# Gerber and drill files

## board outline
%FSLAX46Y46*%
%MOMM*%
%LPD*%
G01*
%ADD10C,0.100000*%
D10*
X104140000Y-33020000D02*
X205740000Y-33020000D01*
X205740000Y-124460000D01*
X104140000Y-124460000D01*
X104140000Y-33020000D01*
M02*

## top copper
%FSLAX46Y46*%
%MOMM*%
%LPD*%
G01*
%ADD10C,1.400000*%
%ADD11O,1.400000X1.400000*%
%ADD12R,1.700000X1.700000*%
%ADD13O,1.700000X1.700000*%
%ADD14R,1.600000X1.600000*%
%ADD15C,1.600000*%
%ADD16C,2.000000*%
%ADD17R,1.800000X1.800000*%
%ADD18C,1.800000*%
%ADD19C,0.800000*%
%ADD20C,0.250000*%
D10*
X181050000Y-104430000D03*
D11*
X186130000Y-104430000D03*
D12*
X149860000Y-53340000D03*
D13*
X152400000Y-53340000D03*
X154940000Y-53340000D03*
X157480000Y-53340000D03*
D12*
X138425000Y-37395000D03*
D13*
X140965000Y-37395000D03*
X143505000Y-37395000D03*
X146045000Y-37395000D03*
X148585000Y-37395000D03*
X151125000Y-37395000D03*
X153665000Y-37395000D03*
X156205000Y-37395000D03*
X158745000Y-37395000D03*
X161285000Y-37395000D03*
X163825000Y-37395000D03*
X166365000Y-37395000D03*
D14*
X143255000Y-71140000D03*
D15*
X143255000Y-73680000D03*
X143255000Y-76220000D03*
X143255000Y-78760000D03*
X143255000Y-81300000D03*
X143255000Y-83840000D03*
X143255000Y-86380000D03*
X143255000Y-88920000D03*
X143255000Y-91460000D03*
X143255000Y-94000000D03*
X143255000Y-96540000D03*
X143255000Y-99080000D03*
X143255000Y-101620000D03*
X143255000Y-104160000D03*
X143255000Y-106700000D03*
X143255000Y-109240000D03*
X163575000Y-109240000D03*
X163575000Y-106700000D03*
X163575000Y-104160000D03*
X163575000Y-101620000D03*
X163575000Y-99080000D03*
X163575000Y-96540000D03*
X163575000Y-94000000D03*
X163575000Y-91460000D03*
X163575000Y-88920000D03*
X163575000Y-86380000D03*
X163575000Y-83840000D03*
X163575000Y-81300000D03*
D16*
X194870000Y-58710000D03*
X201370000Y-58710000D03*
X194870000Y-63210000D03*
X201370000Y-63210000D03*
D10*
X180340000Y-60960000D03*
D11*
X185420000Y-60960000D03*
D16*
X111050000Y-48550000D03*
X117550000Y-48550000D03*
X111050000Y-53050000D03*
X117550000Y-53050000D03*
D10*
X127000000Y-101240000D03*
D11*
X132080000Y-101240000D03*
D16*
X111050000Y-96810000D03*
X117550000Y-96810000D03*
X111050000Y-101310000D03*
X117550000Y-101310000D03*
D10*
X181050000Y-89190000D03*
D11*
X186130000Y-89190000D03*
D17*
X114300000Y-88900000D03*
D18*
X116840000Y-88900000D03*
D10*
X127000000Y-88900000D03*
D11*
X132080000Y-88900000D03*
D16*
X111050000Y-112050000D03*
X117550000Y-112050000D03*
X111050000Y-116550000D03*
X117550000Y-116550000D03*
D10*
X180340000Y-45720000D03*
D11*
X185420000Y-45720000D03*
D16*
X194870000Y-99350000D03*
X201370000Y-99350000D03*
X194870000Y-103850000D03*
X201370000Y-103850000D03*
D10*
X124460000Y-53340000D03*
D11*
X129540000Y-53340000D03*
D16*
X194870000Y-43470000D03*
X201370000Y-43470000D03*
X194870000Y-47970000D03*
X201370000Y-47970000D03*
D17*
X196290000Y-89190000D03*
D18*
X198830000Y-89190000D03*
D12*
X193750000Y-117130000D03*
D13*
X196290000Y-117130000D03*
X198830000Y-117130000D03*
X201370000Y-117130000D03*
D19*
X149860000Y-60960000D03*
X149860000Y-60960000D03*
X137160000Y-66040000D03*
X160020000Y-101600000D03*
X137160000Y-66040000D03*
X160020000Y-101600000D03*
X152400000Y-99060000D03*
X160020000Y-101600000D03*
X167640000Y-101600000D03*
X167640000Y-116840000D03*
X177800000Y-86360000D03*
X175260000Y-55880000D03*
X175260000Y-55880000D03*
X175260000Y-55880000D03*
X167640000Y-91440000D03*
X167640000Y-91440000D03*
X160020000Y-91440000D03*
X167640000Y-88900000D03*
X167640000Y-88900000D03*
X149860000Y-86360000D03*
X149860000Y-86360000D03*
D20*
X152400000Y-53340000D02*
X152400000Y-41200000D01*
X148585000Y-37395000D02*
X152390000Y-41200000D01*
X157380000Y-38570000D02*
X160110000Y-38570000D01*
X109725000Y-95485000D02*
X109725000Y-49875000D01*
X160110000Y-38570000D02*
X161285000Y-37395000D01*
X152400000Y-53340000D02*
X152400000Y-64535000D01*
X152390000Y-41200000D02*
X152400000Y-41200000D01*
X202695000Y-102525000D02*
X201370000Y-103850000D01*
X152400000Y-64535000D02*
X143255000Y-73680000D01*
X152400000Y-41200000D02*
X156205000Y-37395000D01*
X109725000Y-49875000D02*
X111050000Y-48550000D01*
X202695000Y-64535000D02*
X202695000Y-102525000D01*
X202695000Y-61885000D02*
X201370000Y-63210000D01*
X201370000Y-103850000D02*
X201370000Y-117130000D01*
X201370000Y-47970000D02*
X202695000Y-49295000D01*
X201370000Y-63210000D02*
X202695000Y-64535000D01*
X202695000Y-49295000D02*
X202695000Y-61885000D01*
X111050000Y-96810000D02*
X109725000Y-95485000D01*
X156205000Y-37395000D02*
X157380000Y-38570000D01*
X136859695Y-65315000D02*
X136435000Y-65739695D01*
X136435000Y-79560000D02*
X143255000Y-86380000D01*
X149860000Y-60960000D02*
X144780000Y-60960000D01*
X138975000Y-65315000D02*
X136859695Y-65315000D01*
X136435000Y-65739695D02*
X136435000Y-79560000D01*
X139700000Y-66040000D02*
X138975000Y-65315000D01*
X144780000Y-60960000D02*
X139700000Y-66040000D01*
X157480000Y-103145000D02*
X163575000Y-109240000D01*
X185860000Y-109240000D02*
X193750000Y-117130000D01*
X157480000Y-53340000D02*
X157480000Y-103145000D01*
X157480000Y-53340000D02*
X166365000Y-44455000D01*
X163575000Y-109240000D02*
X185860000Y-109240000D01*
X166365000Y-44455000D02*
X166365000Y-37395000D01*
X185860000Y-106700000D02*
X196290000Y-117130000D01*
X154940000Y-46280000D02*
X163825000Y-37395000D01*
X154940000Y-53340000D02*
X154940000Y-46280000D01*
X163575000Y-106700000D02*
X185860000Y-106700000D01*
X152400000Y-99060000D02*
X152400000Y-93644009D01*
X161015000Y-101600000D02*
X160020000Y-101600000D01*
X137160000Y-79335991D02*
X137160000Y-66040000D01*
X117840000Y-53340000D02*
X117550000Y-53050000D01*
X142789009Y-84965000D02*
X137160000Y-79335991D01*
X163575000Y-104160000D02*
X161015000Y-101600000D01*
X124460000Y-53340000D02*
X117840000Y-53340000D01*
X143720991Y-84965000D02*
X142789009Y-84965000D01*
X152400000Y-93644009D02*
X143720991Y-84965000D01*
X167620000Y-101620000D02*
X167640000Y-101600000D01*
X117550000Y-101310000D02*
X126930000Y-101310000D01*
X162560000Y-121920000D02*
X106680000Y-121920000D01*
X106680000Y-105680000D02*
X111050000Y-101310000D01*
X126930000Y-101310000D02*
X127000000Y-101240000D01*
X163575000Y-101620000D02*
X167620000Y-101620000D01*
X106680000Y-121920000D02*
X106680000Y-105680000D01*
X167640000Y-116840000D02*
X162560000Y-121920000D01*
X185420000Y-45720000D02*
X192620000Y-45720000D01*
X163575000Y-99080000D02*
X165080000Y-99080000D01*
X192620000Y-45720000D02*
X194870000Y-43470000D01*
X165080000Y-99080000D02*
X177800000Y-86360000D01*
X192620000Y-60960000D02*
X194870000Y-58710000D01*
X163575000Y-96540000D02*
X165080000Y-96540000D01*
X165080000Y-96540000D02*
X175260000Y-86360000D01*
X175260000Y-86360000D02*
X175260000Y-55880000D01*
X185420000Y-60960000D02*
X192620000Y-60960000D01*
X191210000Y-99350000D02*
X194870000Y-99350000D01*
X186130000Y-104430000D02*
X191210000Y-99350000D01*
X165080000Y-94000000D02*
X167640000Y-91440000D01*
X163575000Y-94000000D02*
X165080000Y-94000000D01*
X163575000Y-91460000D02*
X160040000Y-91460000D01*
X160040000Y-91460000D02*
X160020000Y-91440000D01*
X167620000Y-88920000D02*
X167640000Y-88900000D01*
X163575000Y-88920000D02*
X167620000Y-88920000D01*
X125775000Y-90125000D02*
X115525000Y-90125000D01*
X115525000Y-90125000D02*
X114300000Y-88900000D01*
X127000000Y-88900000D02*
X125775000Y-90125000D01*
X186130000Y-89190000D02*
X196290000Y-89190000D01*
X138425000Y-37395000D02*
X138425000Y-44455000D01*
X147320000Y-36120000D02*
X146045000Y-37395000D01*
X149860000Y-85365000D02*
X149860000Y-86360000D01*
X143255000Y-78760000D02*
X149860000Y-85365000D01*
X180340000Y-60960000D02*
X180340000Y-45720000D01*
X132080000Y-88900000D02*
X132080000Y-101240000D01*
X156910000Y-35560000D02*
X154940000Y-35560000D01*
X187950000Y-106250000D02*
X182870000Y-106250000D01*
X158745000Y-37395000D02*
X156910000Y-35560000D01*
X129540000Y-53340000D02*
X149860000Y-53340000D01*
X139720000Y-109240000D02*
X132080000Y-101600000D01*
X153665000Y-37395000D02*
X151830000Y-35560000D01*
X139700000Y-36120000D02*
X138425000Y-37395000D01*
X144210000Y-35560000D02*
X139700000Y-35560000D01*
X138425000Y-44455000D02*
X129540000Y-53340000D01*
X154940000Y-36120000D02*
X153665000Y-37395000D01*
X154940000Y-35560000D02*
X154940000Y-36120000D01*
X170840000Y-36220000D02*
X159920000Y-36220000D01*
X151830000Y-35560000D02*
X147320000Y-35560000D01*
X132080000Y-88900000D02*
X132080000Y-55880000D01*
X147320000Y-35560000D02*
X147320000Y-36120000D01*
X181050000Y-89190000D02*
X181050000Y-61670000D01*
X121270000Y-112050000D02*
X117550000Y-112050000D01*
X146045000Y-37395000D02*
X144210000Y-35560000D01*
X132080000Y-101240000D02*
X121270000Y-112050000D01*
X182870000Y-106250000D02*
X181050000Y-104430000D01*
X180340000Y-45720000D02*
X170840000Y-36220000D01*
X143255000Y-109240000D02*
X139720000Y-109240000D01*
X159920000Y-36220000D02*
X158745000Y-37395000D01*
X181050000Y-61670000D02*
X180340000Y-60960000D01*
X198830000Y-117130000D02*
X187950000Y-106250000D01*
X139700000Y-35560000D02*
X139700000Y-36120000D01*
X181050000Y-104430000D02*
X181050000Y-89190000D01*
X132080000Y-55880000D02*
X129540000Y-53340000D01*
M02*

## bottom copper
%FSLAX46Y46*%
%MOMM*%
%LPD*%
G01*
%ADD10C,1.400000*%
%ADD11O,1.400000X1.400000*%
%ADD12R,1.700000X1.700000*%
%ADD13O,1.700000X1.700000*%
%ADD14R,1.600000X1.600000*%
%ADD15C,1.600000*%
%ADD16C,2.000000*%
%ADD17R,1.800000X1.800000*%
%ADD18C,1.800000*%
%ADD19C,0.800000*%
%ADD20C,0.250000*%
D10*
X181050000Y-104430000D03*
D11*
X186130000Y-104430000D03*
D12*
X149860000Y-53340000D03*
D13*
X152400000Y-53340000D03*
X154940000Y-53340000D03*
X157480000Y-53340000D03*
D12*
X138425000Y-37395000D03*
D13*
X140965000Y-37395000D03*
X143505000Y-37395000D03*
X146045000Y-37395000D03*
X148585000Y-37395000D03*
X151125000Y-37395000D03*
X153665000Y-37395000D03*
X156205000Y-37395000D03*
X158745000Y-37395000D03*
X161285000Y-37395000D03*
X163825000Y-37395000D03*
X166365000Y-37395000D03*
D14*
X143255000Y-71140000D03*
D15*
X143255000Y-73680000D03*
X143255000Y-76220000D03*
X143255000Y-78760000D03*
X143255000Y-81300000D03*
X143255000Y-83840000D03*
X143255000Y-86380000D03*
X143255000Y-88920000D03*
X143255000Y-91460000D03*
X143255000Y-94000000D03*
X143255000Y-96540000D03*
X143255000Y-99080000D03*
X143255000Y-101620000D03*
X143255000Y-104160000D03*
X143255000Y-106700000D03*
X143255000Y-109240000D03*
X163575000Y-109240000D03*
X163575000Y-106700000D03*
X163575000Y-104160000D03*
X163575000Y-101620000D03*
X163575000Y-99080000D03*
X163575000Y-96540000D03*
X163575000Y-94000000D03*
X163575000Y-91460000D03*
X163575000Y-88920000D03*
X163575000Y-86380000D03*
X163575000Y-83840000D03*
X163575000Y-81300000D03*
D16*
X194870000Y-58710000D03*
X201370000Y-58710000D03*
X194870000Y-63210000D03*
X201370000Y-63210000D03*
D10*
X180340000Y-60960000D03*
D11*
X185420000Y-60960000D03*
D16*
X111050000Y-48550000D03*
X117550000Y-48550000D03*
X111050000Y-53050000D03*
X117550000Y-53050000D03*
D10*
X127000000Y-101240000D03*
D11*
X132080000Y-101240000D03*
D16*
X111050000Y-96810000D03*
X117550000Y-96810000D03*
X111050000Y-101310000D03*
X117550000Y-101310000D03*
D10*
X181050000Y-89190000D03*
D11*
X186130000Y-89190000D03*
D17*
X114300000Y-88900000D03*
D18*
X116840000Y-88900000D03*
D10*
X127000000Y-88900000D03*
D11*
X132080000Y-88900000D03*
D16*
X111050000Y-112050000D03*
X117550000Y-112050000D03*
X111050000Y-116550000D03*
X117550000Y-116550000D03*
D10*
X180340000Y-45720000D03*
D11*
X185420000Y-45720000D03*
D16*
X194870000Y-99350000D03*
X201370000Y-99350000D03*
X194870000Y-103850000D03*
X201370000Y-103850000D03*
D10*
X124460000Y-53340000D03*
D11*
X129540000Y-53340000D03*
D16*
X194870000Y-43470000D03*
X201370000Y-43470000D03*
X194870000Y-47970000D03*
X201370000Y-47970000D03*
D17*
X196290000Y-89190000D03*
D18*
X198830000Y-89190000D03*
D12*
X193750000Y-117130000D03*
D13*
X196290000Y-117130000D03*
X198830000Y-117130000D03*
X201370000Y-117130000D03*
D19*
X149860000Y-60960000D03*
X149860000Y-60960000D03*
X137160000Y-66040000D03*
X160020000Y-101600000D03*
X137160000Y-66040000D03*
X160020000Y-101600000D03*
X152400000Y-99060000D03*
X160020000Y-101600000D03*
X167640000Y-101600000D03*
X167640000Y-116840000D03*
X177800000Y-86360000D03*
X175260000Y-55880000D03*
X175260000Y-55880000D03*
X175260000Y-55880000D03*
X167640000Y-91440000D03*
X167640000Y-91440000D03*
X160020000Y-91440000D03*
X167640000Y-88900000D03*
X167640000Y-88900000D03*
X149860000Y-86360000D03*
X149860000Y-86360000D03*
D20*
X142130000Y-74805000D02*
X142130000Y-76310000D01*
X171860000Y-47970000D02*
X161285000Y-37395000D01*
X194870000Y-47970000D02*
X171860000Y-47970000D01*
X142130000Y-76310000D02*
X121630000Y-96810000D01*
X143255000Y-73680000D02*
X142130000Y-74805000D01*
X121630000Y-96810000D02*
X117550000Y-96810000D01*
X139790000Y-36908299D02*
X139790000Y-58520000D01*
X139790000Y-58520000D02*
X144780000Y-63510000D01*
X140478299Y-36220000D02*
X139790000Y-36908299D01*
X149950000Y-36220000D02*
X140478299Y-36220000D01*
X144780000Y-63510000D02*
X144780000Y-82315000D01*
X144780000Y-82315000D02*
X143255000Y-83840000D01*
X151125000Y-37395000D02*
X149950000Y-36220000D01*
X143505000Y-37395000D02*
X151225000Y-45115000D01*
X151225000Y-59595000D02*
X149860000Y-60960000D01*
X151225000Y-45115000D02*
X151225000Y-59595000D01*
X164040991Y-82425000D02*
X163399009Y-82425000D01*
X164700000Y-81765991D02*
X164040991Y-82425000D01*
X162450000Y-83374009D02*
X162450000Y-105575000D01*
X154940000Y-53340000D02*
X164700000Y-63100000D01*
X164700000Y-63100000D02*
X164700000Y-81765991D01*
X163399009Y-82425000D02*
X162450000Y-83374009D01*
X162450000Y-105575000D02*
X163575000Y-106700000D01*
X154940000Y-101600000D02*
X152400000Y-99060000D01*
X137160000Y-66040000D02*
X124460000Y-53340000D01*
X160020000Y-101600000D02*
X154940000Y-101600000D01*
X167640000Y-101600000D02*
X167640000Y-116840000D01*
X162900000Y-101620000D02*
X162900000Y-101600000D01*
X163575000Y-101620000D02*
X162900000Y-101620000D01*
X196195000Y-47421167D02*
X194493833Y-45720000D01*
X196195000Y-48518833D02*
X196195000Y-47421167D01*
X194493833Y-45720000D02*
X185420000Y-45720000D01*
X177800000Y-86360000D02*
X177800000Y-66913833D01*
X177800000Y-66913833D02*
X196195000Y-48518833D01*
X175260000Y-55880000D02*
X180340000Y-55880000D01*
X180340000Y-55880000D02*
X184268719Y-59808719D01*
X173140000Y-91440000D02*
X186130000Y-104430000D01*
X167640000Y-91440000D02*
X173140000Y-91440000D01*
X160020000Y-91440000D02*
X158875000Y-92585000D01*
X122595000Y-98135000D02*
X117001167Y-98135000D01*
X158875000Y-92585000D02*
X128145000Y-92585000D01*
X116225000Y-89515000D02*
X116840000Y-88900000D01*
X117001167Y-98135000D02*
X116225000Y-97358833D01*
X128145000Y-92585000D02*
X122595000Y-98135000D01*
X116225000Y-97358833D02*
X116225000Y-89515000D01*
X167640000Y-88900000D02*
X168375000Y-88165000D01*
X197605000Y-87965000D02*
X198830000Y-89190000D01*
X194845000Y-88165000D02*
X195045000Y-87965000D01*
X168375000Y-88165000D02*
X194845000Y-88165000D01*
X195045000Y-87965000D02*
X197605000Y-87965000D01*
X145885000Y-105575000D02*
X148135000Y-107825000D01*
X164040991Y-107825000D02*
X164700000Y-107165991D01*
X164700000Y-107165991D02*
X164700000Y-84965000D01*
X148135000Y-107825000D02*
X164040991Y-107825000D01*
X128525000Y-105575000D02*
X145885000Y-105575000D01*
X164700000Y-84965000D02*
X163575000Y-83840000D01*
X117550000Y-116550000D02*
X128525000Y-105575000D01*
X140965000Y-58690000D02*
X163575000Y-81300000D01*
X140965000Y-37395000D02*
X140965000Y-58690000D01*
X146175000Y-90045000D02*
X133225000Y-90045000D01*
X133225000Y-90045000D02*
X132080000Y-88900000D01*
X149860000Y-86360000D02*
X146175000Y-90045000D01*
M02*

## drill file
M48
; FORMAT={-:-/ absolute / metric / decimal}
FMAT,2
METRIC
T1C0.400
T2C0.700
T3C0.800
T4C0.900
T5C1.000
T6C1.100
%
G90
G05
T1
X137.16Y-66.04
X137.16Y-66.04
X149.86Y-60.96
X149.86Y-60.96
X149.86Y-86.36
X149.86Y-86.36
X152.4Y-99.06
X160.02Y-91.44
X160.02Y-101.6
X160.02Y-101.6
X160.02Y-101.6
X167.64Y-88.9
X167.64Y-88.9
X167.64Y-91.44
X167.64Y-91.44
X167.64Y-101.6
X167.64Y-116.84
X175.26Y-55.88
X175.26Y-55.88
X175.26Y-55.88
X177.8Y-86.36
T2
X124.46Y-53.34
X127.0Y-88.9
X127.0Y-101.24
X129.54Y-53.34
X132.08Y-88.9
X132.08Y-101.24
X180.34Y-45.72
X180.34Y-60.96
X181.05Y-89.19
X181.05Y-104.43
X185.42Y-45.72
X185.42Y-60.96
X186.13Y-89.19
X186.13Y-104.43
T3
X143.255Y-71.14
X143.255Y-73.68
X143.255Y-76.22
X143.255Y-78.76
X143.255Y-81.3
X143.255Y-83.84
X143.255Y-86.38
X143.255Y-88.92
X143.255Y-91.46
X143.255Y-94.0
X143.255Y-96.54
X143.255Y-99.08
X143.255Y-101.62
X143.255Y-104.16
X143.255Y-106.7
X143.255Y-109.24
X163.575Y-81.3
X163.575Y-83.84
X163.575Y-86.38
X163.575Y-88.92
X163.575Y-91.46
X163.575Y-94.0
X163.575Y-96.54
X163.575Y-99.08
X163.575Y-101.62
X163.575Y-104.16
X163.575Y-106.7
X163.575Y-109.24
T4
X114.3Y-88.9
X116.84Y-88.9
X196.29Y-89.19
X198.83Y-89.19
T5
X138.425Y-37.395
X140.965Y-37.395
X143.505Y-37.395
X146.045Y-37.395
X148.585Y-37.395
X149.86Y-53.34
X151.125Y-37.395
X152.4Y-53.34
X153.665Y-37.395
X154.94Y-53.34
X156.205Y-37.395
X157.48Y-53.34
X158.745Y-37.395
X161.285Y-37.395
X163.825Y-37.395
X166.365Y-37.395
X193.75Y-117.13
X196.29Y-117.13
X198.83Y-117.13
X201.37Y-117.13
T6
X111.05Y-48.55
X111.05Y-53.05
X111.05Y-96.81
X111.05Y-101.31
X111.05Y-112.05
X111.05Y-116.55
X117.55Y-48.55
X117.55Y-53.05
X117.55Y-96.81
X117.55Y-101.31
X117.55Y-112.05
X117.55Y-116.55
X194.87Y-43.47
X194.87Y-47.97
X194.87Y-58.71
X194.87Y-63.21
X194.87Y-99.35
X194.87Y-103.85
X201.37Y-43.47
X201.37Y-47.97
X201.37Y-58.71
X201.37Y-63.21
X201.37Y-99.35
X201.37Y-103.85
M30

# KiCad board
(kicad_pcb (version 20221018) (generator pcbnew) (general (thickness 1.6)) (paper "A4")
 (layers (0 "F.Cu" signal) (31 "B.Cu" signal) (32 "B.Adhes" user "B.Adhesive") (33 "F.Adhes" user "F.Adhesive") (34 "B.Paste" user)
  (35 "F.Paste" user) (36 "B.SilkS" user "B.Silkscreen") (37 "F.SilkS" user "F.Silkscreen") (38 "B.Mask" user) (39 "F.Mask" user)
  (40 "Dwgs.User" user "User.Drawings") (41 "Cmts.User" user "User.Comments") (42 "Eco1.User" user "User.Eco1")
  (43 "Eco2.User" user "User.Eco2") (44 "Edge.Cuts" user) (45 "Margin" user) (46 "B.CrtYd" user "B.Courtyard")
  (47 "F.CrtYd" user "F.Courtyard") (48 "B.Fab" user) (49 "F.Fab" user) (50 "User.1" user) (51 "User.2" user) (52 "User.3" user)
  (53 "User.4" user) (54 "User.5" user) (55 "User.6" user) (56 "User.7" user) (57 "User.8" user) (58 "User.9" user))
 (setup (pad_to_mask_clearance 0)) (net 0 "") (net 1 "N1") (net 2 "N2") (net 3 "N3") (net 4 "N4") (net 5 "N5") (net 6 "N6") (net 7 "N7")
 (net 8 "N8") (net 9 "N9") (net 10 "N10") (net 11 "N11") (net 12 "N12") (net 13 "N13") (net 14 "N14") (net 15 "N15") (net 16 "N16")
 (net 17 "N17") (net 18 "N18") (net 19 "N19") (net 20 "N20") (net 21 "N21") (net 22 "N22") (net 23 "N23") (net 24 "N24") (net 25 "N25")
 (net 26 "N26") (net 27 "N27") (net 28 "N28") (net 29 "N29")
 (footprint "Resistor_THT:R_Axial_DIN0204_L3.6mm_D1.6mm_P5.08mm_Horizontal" (layer "F.Cu") (at 181.05 104.43)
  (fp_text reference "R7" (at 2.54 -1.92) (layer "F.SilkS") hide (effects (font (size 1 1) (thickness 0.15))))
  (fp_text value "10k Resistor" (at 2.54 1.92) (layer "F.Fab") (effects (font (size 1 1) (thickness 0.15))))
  (pad "1" thru_hole circle (at 0 0) (size 1.4 1.4) (drill 0.7) (layers "*.Cu" "*.Mask") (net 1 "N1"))
  (pad "2" thru_hole oval (at 5.08 0) (size 1.4 1.4) (drill 0.7) (layers "*.Cu" "*.Mask") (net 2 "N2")))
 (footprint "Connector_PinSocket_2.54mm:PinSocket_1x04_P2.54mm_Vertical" (layer "F.Cu") (at 149.86 53.34 90)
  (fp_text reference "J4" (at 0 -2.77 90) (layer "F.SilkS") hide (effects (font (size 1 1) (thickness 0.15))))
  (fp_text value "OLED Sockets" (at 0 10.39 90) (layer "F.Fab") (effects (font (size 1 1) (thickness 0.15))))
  (pad "1" thru_hole rect (at 0 0 90) (size 1.7 1.7) (drill 1) (layers "*.Cu" "*.Mask") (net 1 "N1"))
  (pad "2" thru_hole oval (at 0 2.54 90) (size 1.7 1.7) (drill 1) (layers "*.Cu" "*.Mask") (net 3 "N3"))
  (pad "3" thru_hole oval (at 0 5.08 90) (size 1.7 1.7) (drill 1) (layers "*.Cu" "*.Mask") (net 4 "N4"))
  (pad "4" thru_hole oval (at 0 7.62 90) (size 1.7 1.7) (drill 1) (layers "*.Cu" "*.Mask") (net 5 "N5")))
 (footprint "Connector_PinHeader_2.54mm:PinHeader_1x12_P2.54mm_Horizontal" (layer "F.Cu") (at 138.425 37.395 90)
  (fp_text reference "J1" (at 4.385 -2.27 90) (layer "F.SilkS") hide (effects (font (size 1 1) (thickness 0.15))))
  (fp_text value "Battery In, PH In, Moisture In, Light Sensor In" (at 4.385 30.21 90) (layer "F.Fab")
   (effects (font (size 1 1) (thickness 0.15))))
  (pad "1" thru_hole rect (at 0 0 90) (size 1.7 1.7) (drill 1) (layers "*.Cu" "*.Mask") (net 1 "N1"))
  (pad "2" thru_hole oval (at 0 2.54 90) (size 1.7 1.7) (drill 1) (layers "*.Cu" "*.Mask") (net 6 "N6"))
  (pad "3" thru_hole oval (at 0 5.08 90) (size 1.7 1.7) (drill 1) (layers "*.Cu" "*.Mask") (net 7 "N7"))
  (pad "4" thru_hole oval (at 0 7.62 90) (size 1.7 1.7) (drill 1) (layers "*.Cu" "*.Mask") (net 1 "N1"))
  (pad "5" thru_hole oval (at 0 10.16 90) (size 1.7 1.7) (drill 1) (layers "*.Cu" "*.Mask") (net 3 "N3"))
  (pad "6" thru_hole oval (at 0 12.7 90) (size 1.7 1.7) (drill 1) (layers "*.Cu" "*.Mask") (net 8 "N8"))
  (pad "7" thru_hole oval (at 0 15.24 90) (size 1.7 1.7) (drill 1) (layers "*.Cu" "*.Mask") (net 1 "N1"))
  (pad "8" thru_hole oval (at 0 17.78 90) (size 1.7 1.7) (drill 1) (layers "*.Cu" "*.Mask") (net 3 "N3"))
  (pad "9" thru_hole oval (at 0 20.32 90) (size 1.7 1.7) (drill 1) (layers "*.Cu" "*.Mask") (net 1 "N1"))
  (pad "10" thru_hole oval (at 0 22.86 90) (size 1.7 1.7) (drill 1) (layers "*.Cu" "*.Mask") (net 3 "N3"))
  (pad "11" thru_hole oval (at 0 25.4 90) (size 1.7 1.7) (drill 1) (layers "*.Cu" "*.Mask") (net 4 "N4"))
  (pad "12" thru_hole oval (at 0 27.94 90) (size 1.7 1.7) (drill 1) (layers "*.Cu" "*.Mask") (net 5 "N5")))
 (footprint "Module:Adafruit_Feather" (layer "F.Cu") (at 143.255 71.14)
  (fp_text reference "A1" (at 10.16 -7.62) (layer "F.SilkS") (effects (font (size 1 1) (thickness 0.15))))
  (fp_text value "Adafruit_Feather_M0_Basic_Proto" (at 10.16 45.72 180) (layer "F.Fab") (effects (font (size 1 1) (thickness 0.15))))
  (pad "1" thru_hole rect (at 0 0 180) (size 1.6 1.6) (drill 0.8) (layers "*.Cu" "*.Mask") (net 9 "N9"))
  (pad "2" thru_hole circle (at 0 2.54 180) (size 1.6 1.6) (drill 0.8) (layers "*.Cu" "*.Mask") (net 3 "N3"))
  (pad "3" thru_hole circle (at 0 5.08 180) (size 1.6 1.6) (drill 0.8) (layers "*.Cu" "*.Mask") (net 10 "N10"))
  (pad "4" thru_hole circle (at 0 7.62 180) (size 1.6 1.6) (drill 0.8) (layers "*.Cu" "*.Mask") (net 1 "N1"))
  (pad "5" thru_hole circle (at 0 10.16 180) (size 1.6 1.6) (drill 0.8) (layers "*.Cu" "*.Mask") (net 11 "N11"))
  (pad "6" thru_hole circle (at 0 12.7 180) (size 1.6 1.6) (drill 0.8) (layers "*.Cu" "*.Mask") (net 8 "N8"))
  (pad "7" thru_hole circle (at 0 15.24 180) (size 1.6 1.6) (drill 0.8) (layers "*.Cu" "*.Mask") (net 7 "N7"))
  (pad "8" thru_hole circle (at 0 17.78 180) (size 1.6 1.6) (drill 0.8) (layers "*.Cu" "*.Mask") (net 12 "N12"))
  (pad "9" thru_hole circle (at 0 20.32 180) (size 1.6 1.6) (drill 0.8) (layers "*.Cu" "*.Mask") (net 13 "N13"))
  (pad "10" thru_hole circle (at 0 22.86 180) (size 1.6 1.6) (drill 0.8) (layers "*.Cu" "*.Mask") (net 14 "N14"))
  (pad "11" thru_hole circle (at 0 25.4 180) (size 1.6 1.6) (drill 0.8) (layers "*.Cu" "*.Mask") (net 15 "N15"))
  (pad "12" thru_hole circle (at 0 27.94 180) (size 1.6 1.6) (drill 0.8) (layers "*.Cu" "*.Mask") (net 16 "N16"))
  (pad "13" thru_hole circle (at 0 30.48 180) (size 1.6 1.6) (drill 0.8) (layers "*.Cu" "*.Mask") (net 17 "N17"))
  (pad "14" thru_hole circle (at 0 33.02 180) (size 1.6 1.6) (drill 0.8) (layers "*.Cu" "*.Mask") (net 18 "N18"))
  (pad "15" thru_hole circle (at 0 35.56 180) (size 1.6 1.6) (drill 0.8) (layers "*.Cu" "*.Mask") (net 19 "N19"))
  (pad "16" thru_hole circle (at 0 38.1 180) (size 1.6 1.6) (drill 0.8) (layers "*.Cu" "*.Mask") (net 1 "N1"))
  (pad "17" thru_hole circle (at 20.32 38.1 180) (size 1.6 1.6) (drill 0.8) (layers "*.Cu" "*.Mask") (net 5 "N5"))
  (pad "18" thru_hole circle (at 20.32 35.56 180) (size 1.6 1.6) (drill 0.8) (layers "*.Cu" "*.Mask") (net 4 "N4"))
  (pad "19" thru_hole circle (at 20.32 33.02 180) (size 1.6 1.6) (drill 0.8) (layers "*.Cu" "*.Mask") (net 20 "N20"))
  (pad "20" thru_hole circle (at 20.32 30.48 180) (size 1.6 1.6) (drill 0.8) (layers "*.Cu" "*.Mask") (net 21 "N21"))
  (pad "21" thru_hole circle (at 20.32 27.94 180) (size 1.6 1.6) (drill 0.8) (layers "*.Cu" "*.Mask") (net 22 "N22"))
  (pad "22" thru_hole circle (at 20.32 25.4 180) (size 1.6 1.6) (drill 0.8) (layers "*.Cu" "*.Mask") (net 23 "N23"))
  (pad "23" thru_hole circle (at 20.32 22.86 180) (size 1.6 1.6) (drill 0.8) (layers "*.Cu" "*.Mask") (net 2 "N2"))
  (pad "24" thru_hole circle (at 20.32 20.32 180) (size 1.6 1.6) (drill 0.8) (layers "*.Cu" "*.Mask") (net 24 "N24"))
  (pad "25" thru_hole circle (at 20.32 17.78 180) (size 1.6 1.6) (drill 0.8) (layers "*.Cu" "*.Mask") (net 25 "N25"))
  (pad "26" thru_hole circle (at 20.32 15.24 180) (size 1.6 1.6) (drill 0.8) (layers "*.Cu" "*.Mask") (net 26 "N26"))
  (pad "27" thru_hole circle (at 20.32 12.7 180) (size 1.6 1.6) (drill 0.8) (layers "*.Cu" "*.Mask") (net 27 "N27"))
  (pad "28" thru_hole circle (at 20.32 10.16 180) (size 1.6 1.6) (drill 0.8) (layers "*.Cu" "*.Mask") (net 6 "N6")))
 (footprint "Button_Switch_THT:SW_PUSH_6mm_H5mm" (layer "F.Cu") (at 194.87 58.71)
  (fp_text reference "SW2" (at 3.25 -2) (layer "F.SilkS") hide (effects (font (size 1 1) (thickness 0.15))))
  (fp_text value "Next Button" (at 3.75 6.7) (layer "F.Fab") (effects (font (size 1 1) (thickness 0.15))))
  (pad "1" thru_hole circle (at 0 0 90) (size 2 2) (drill 1.1) (layers "*.Cu" "*.Mask") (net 23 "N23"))
  (pad "1" thru_hole circle (at 6.5 0 90) (size 2 2) (drill 1.1) (layers "*.Cu" "*.Mask") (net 23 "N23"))
  (pad "2" thru_hole circle (at 0 4.5 90) (size 2 2) (drill 1.1) (layers "*.Cu" "*.Mask") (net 3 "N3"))
  (pad "2" thru_hole circle (at 6.5 4.5 90) (size 2 2) (drill 1.1) (layers "*.Cu" "*.Mask") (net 3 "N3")))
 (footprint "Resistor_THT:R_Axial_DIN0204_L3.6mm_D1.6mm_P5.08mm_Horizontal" (layer "F.Cu") (at 180.34 60.96)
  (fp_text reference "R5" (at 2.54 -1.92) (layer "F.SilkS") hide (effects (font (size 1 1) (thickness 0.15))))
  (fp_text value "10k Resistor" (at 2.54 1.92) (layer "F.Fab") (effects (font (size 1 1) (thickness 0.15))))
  (pad "1" thru_hole circle (at 0 0) (size 1.4 1.4) (drill 0.7) (layers "*.Cu" "*.Mask") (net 1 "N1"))
  (pad "2" thru_hole oval (at 5.08 0) (size 1.4 1.4) (drill 0.7) (layers "*.Cu" "*.Mask") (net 23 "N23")))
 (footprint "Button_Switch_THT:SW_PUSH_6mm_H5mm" (layer "F.Cu") (at 111.05 48.55)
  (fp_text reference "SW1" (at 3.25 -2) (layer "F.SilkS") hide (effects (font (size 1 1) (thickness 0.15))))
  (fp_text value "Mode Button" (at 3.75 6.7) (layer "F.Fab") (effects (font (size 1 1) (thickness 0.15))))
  (pad "1" thru_hole circle (at 0 0 90) (size 2 2) (drill 1.1) (layers "*.Cu" "*.Mask") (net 3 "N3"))
  (pad "1" thru_hole circle (at 6.5 0 90) (size 2 2) (drill 1.1) (layers "*.Cu" "*.Mask") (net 3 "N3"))
  (pad "2" thru_hole circle (at 0 4.5 90) (size 2 2) (drill 1.1) (layers "*.Cu" "*.Mask") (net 20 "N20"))
  (pad "2" thru_hole circle (at 6.5 4.5 90) (size 2 2) (drill 1.1) (layers "*.Cu" "*.Mask") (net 20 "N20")))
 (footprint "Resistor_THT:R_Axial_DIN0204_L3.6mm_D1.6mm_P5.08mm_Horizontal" (layer "F.Cu") (at 127 101.24)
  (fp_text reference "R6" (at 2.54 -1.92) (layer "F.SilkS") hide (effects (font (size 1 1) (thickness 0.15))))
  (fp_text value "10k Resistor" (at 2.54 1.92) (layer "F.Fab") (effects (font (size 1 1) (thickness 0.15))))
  (pad "1" thru_hole circle (at 0 0) (size 1.4 1.4) (drill 0.7) (layers "*.Cu" "*.Mask") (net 21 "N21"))
  (pad "2" thru_hole oval (at 5.08 0) (size 1.4 1.4) (drill 0.7) (layers "*.Cu" "*.Mask") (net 1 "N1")))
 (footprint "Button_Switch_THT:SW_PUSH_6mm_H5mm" (layer "F.Cu") (at 111.05 96.81)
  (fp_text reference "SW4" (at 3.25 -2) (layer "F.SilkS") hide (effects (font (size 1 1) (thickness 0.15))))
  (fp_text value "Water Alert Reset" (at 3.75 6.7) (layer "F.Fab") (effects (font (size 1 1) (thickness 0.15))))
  (pad "1" thru_hole circle (at 0 0 90) (size 2 2) (drill 1.1) (layers "*.Cu" "*.Mask") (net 3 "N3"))
  (pad "1" thru_hole circle (at 6.5 0 90) (size 2 2) (drill 1.1) (layers "*.Cu" "*.Mask") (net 3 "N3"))
  (pad "2" thru_hole circle (at 0 4.5 90) (size 2 2) (drill 1.1) (layers "*.Cu" "*.Mask") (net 21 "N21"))
  (pad "2" thru_hole circle (at 6.5 4.5 90) (size 2 2) (drill 1.1) (layers "*.Cu" "*.Mask") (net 21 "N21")))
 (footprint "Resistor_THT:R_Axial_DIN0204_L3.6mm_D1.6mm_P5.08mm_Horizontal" (layer "F.Cu") (at 181.05 89.19)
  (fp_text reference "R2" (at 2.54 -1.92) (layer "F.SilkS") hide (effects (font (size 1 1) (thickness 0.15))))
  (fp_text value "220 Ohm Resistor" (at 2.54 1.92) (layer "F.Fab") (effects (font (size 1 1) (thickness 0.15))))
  (pad "1" thru_hole circle (at 0 0) (size 1.4 1.4) (drill 0.7) (layers "*.Cu" "*.Mask") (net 1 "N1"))
  (pad "2" thru_hole oval (at 5.08 0) (size 1.4 1.4) (drill 0.7) (layers "*.Cu" "*.Mask") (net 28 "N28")))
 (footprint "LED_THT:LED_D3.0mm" (layer "F.Cu") (at 114.3 88.9)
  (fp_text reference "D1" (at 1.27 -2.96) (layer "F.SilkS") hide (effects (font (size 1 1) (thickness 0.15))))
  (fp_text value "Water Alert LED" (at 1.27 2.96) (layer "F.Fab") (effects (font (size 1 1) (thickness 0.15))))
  (pad "1" thru_hole rect (at 0 0) (size 1.8 1.8) (drill 0.9) (layers "*.Cu" "*.Mask") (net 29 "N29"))
  (pad "2" thru_hole circle (at 2.54 0) (size 1.8 1.8) (drill 0.9) (layers "*.Cu" "*.Mask") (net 24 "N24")))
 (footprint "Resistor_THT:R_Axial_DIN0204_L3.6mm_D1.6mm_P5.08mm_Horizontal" (layer "F.Cu") (at 127 88.9)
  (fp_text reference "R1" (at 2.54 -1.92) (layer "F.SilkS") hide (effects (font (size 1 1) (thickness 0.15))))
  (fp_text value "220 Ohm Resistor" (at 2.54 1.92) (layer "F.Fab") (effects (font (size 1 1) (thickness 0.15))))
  (pad "1" thru_hole circle (at 0 0) (size 1.4 1.4) (drill 0.7) (layers "*.Cu" "*.Mask") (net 29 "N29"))
  (pad "2" thru_hole oval (at 5.08 0) (size 1.4 1.4) (drill 0.7) (layers "*.Cu" "*.Mask") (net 1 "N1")))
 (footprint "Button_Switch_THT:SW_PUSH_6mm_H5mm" (layer "F.Cu") (at 111.05 112.05)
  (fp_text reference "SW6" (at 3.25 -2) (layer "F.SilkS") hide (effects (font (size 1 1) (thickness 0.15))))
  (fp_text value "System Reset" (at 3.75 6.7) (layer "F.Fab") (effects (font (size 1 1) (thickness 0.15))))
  (pad "1" thru_hole circle (at 0 0 90) (size 2 2) (drill 1.1) (layers "*.Cu" "*.Mask") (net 1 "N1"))
  (pad "1" thru_hole circle (at 6.5 0 90) (size 2 2) (drill 1.1) (layers "*.Cu" "*.Mask") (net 1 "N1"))
  (pad "2" thru_hole circle (at 0 4.5 90) (size 2 2) (drill 1.1) (layers "*.Cu" "*.Mask") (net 27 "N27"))
  (pad "2" thru_hole circle (at 6.5 4.5 90) (size 2 2) (drill 1.1) (layers "*.Cu" "*.Mask") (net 27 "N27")))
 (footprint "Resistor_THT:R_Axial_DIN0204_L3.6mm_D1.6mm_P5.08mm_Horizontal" (layer "F.Cu") (at 180.34 45.72)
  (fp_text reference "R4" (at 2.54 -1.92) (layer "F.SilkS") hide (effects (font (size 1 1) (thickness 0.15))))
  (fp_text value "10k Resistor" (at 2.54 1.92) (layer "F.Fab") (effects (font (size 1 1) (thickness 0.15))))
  (pad "1" thru_hole circle (at 0 0) (size 1.4 1.4) (drill 0.7) (layers "*.Cu" "*.Mask") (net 1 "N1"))
  (pad "2" thru_hole oval (at 5.08 0) (size 1.4 1.4) (drill 0.7) (layers "*.Cu" "*.Mask") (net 22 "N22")))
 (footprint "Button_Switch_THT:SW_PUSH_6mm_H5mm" (layer "F.Cu") (at 194.87 99.35)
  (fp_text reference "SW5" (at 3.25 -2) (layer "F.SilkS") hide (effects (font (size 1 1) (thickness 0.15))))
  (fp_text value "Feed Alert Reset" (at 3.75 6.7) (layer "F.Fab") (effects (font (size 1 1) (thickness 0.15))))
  (pad "1" thru_hole circle (at 0 0 90) (size 2 2) (drill 1.1) (layers "*.Cu" "*.Mask") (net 2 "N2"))
  (pad "1" thru_hole circle (at 6.5 0 90) (size 2 2) (drill 1.1) (layers "*.Cu" "*.Mask") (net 2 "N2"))
  (pad "2" thru_hole circle (at 0 4.5 90) (size 2 2) (drill 1.1) (layers "*.Cu" "*.Mask") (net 3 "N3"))
  (pad "2" thru_hole circle (at 6.5 4.5 90) (size 2 2) (drill 1.1) (layers "*.Cu" "*.Mask") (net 3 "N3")))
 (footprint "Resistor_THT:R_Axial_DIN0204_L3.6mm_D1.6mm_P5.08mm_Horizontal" (layer "F.Cu") (at 124.46 53.34)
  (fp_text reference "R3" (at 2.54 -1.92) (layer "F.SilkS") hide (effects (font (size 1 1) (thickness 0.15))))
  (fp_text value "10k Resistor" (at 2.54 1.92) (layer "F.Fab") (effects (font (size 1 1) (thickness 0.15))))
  (pad "1" thru_hole circle (at 0 0) (size 1.4 1.4) (drill 0.7) (layers "*.Cu" "*.Mask") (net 20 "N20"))
  (pad "2" thru_hole oval (at 5.08 0) (size 1.4 1.4) (drill 0.7) (layers "*.Cu" "*.Mask") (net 1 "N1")))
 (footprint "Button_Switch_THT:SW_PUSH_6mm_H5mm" (layer "F.Cu") (at 194.87 43.47)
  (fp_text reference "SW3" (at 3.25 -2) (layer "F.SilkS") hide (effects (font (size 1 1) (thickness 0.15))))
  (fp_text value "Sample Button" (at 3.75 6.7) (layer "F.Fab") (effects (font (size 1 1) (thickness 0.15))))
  (pad "1" thru_hole circle (at 0 0 90) (size 2 2) (drill 1.1) (layers "*.Cu" "*.Mask") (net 22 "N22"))
  (pad "1" thru_hole circle (at 6.5 0 90) (size 2 2) (drill 1.1) (layers "*.Cu" "*.Mask") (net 22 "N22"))
  (pad "2" thru_hole circle (at 0 4.5 90) (size 2 2) (drill 1.1) (layers "*.Cu" "*.Mask") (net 3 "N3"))
  (pad "2" thru_hole circle (at 6.5 4.5 90) (size 2 2) (drill 1.1) (layers "*.Cu" "*.Mask") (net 3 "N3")))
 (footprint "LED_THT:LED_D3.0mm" (layer "F.Cu") (at 196.29 89.19)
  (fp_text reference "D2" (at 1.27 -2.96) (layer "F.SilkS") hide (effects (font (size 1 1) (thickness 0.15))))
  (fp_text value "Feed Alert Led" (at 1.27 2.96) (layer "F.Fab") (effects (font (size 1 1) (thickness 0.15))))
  (pad "1" thru_hole rect (at 0 0) (size 1.8 1.8) (drill 0.9) (layers "*.Cu" "*.Mask") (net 28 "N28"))
  (pad "2" thru_hole circle (at 2.54 0) (size 1.8 1.8) (drill 0.9) (layers "*.Cu" "*.Mask") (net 25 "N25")))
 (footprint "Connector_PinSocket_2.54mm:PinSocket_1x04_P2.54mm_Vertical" (layer "F.Cu") (at 193.75 117.13 90)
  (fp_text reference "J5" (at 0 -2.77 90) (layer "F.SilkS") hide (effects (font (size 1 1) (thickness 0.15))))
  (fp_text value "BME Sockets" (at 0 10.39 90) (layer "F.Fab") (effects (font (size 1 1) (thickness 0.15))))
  (pad "1" thru_hole rect (at 0 0 90) (size 1.7 1.7) (drill 1) (layers "*.Cu" "*.Mask") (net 5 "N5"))
  (pad "2" thru_hole oval (at 0 2.54 90) (size 1.7 1.7) (drill 1) (layers "*.Cu" "*.Mask") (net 4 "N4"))
  (pad "3" thru_hole oval (at 0 5.08 90) (size 1.7 1.7) (drill 1) (layers "*.Cu" "*.Mask") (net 1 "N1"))
  (pad "4" thru_hole oval (at 0 7.62 90) (size 1.7 1.7) (drill 1) (layers "*.Cu" "*.Mask") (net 3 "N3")))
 (gr_rect (start 104.14 33.02) (end 205.74 124.46) (stroke (width 0.1) (type default)) (fill none) (layer "Edge.Cuts"))
 (segment (start 152.4 53.34) (end 152.4 41.2) (width 0.25) (layer "F.Cu") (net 3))
 (segment (start 148.585 37.395) (end 152.39 41.2) (width 0.25) (layer "F.Cu") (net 3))
 (segment (start 157.38 38.57) (end 160.11 38.57) (width 0.25) (layer "F.Cu") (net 3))
 (segment (start 109.725 95.485) (end 109.725 49.875) (width 0.25) (layer "F.Cu") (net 3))
 (segment (start 160.11 38.57) (end 161.285 37.395) (width 0.25) (layer "F.Cu") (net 3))
 (segment (start 152.4 53.34) (end 152.4 64.535) (width 0.25) (layer "F.Cu") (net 3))
 (segment (start 152.39 41.2) (end 152.4 41.2) (width 0.25) (layer "F.Cu") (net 3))
 (segment (start 202.695 102.525) (end 201.37 103.85) (width 0.25) (layer "F.Cu") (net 3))
 (segment (start 152.4 64.535) (end 143.255 73.68) (width 0.25) (layer "F.Cu") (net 3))
 (segment (start 152.4 41.2) (end 156.205 37.395) (width 0.25) (layer "F.Cu") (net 3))
 (segment (start 109.725 49.875) (end 111.05 48.55) (width 0.25) (layer "F.Cu") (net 3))
 (segment (start 202.695 64.535) (end 202.695 102.525) (width 0.25) (layer "F.Cu") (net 3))
 (segment (start 202.695 61.885) (end 201.37 63.21) (width 0.25) (layer "F.Cu") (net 3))
 (segment (start 201.37 103.85) (end 201.37 117.13) (width 0.25) (layer "F.Cu") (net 3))
 (segment (start 201.37 47.97) (end 202.695 49.295) (width 0.25) (layer "F.Cu") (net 3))
 (segment (start 201.37 63.21) (end 202.695 64.535) (width 0.25) (layer "F.Cu") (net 3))
 (segment (start 202.695 49.295) (end 202.695 61.885) (width 0.25) (layer "F.Cu") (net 3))
 (segment (start 111.05 96.81) (end 109.725 95.485) (width 0.25) (layer "F.Cu") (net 3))
 (segment (start 156.205 37.395) (end 157.38 38.57) (width 0.25) (layer "F.Cu") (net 3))
 (segment (start 142.13 74.805) (end 142.13 76.31) (width 0.25) (layer "B.Cu") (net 3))
 (segment (start 171.86 47.97) (end 161.285 37.395) (width 0.25) (layer "B.Cu") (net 3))
 (segment (start 194.87 47.97) (end 171.86 47.97) (width 0.25) (layer "B.Cu") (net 3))
 (segment (start 142.13 76.31) (end 121.63 96.81) (width 0.25) (layer "B.Cu") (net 3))
 (segment (start 143.255 73.68) (end 142.13 74.805) (width 0.25) (layer "B.Cu") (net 3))
 (segment (start 121.63 96.81) (end 117.55 96.81) (width 0.25) (layer "B.Cu") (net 3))
 (segment (start 139.79 36.908299) (end 139.79 58.52) (width 0.25) (layer "B.Cu") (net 8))
 (segment (start 139.79 58.52) (end 144.78 63.51) (width 0.25) (layer "B.Cu") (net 8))
 (segment (start 140.478299 36.22) (end 139.79 36.908299) (width 0.25) (layer "B.Cu") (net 8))
 (segment (start 149.95 36.22) (end 140.478299 36.22) (width 0.25) (layer "B.Cu") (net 8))
 (segment (start 144.78 63.51) (end 144.78 82.315) (width 0.25) (layer "B.Cu") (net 8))
 (segment (start 144.78 82.315) (end 143.255 83.84) (width 0.25) (layer "B.Cu") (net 8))
 (segment (start 151.125 37.395) (end 149.95 36.22) (width 0.25) (layer "B.Cu") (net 8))
 (segment (start 136.859695 65.315) (end 136.435 65.739695) (width 0.25) (layer "F.Cu") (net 7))
 (segment (start 136.435 79.56) (end 143.255 86.38) (width 0.25) (layer "F.Cu") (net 7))
 (segment (start 149.86 60.96) (end 144.78 60.96) (width 0.25) (layer "F.Cu") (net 7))
 (segment (start 138.975 65.315) (end 136.859695 65.315) (width 0.25) (layer "F.Cu") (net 7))
 (segment (start 136.435 65.739695) (end 136.435 79.56) (width 0.25) (layer "F.Cu") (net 7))
 (segment (start 139.7 66.04) (end 138.975 65.315) (width 0.25) (layer "F.Cu") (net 7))
 (segment (start 144.78 60.96) (end 139.7 66.04) (width 0.25) (layer "F.Cu") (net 7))
 (via (at 149.86 60.96) (size 0.8) (drill 0.4) (layers "F.Cu" "B.Cu") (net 7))
 (via (at 149.86 60.96) (size 0.8) (drill 0.4) (layers "F.Cu" "B.Cu") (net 7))
 (segment (start 143.505 37.395) (end 151.225 45.115) (width 0.25) (layer "B.Cu") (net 7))
 (segment (start 151.225 59.595) (end 149.86 60.96) (width 0.25) (layer "B.Cu") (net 7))
 (segment (start 151.225 45.115) (end 151.225 59.595) (width 0.25) (layer "B.Cu") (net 7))
 (segment (start 157.48 103.145) (end 163.575 109.24) (width 0.25) (layer "F.Cu") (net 5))
 (segment (start 185.86 109.24) (end 193.75 117.13) (width 0.25) (layer "F.Cu") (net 5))
 (segment (start 157.48 53.34) (end 157.48 103.145) (width 0.25) (layer "F.Cu") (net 5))
 (segment (start 157.48 53.34) (end 166.365 44.455) (width 0.25) (layer "F.Cu") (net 5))
 (segment (start 163.575 109.24) (end 185.86 109.24) (width 0.25) (layer "F.Cu") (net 5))
 (segment (start 166.365 44.455) (end 166.365 37.395) (width 0.25) (layer "F.Cu") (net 5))
 (segment (start 185.86 106.7) (end 196.29 117.13) (width 0.25) (layer "F.Cu") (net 4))
 (segment (start 154.94 46.28) (end 163.825 37.395) (width 0.25) (layer "F.Cu") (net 4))
 (segment (start 154.94 53.34) (end 154.94 46.28) (width 0.25) (layer "F.Cu") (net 4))
 (segment (start 163.575 106.7) (end 185.86 106.7) (width 0.25) (layer "F.Cu") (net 4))
 (segment (start 164.040991 82.425) (end 163.399009 82.425) (width 0.25) (layer "B.Cu") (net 4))
 (segment (start 164.7 81.765991) (end 164.040991 82.425) (width 0.25) (layer "B.Cu") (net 4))
 (segment (start 162.45 83.374009) (end 162.45 105.575) (width 0.25) (layer "B.Cu") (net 4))
 (segment (start 154.94 53.34) (end 164.7 63.1) (width 0.25) (layer "B.Cu") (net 4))
 (segment (start 164.7 63.1) (end 164.7 81.765991) (width 0.25) (layer "B.Cu") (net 4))
 (segment (start 163.399009 82.425) (end 162.45 83.374009) (width 0.25) (layer "B.Cu") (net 4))
 (segment (start 162.45 105.575) (end 163.575 106.7) (width 0.25) (layer "B.Cu") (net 4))
 (segment (start 152.4 99.06) (end 152.4 93.644009) (width 0.25) (layer "F.Cu") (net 20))
 (segment (start 161.015 101.6) (end 160.02 101.6) (width 0.25) (layer "F.Cu") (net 20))
 (segment (start 137.16 79.335991) (end 137.16 66.04) (width 0.25) (layer "F.Cu") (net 20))
 (segment (start 117.84 53.34) (end 117.55 53.05) (width 0.25) (layer "F.Cu") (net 20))
 (segment (start 142.789009 84.965) (end 137.16 79.335991) (width 0.25) (layer "F.Cu") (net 20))
 (segment (start 163.575 104.16) (end 161.015 101.6) (width 0.25) (layer "F.Cu") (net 20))
 (segment (start 124.46 53.34) (end 117.84 53.34) (width 0.25) (layer "F.Cu") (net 20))
 (segment (start 143.720991 84.965) (end 142.789009 84.965) (width 0.25) (layer "F.Cu") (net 20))
 (segment (start 152.4 93.644009) (end 143.720991 84.965) (width 0.25) (layer "F.Cu") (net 20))
 (via (at 137.16 66.04) (size 0.8) (drill 0.4) (layers "F.Cu" "B.Cu") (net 20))
 (via (at 160.02 101.6) (size 0.8) (drill 0.4) (layers "F.Cu" "B.Cu") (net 20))
 (via (at 137.16 66.04) (size 0.8) (drill 0.4) (layers "F.Cu" "B.Cu") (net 20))
 (via (at 160.02 101.6) (size 0.8) (drill 0.4) (layers "F.Cu" "B.Cu") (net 20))
 (via (at 152.4 99.06) (size 0.8) (drill 0.4) (layers "F.Cu" "B.Cu") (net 20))
 (via (at 160.02 101.6) (size 0.8) (drill 0.4) (layers "F.Cu" "B.Cu") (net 20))
 (segment (start 154.94 101.6) (end 152.4 99.06) (width 0.25) (layer "B.Cu") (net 20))
 (segment (start 137.16 66.04) (end 124.46 53.34) (width 0.25) (layer "B.Cu") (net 20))
 (segment (start 160.02 101.6) (end 154.94 101.6) (width 0.25) (layer "B.Cu") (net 20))
 (segment (start 167.62 101.62) (end 167.64 101.6) (width 0.25) (layer "F.Cu") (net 21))
 (segment (start 117.55 101.31) (end 126.93 101.31) (width 0.25) (layer "F.Cu") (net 21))
 (segment (start 162.56 121.92) (end 106.68 121.92) (width 0.25) (layer "F.Cu") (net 21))
 (segment (start 106.68 105.68) (end 111.05 101.31) (width 0.25) (layer "F.Cu") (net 21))
 (segment (start 126.93 101.31) (end 127 101.24) (width 0.25) (layer "F.Cu") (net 21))
 (segment (start 163.575 101.62) (end 167.62 101.62) (width 0.25) (layer "F.Cu") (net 21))
 (segment (start 106.68 121.92) (end 106.68 105.68) (width 0.25) (layer "F.Cu") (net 21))
 (segment (start 167.64 116.84) (end 162.56 121.92) (width 0.25) (layer "F.Cu") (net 21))
 (via (at 167.64 101.6) (size 0.8) (drill 0.4) (layers "F.Cu" "B.Cu") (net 21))
 (via (at 167.64 116.84) (size 0.8) (drill 0.4) (layers "F.Cu" "B.Cu") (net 21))
 (segment (start 167.64 101.6) (end 167.64 116.84) (width 0.25) (layer "B.Cu") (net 21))
 (segment (start 162.9 101.62) (end 162.9 101.6) (width 0.25) (layer "B.Cu") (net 21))
 (segment (start 163.575 101.62) (end 162.9 101.62) (width 0.25) (layer "B.Cu") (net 21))
 (segment (start 185.42 45.72) (end 192.62 45.72) (width 0.25) (layer "F.Cu") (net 22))
 (segment (start 163.575 99.08) (end 165.08 99.08) (width 0.25) (layer "F.Cu") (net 22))
 (segment (start 192.62 45.72) (end 194.87 43.47) (width 0.25) (layer "F.Cu") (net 22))
 (segment (start 165.08 99.08) (end 177.8 86.36) (width 0.25) (layer "F.Cu") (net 22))
 (via (at 177.8 86.36) (size 0.8) (drill 0.4) (layers "F.Cu" "B.Cu") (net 22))
 (segment (start 196.195 47.421167) (end 194.493833 45.72) (width 0.25) (layer "B.Cu") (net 22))
 (segment (start 196.195 48.518833) (end 196.195 47.421167) (width 0.25) (layer "B.Cu") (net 22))
 (segment (start 194.493833 45.72) (end 185.42 45.72) (width 0.25) (layer "B.Cu") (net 22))
 (segment (start 177.8 86.36) (end 177.8 66.913833) (width 0.25) (layer "B.Cu") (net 22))
 (segment (start 177.8 66.913833) (end 196.195 48.518833) (width 0.25) (layer "B.Cu") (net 22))
 (segment (start 192.62 60.96) (end 194.87 58.71) (width 0.25) (layer "F.Cu") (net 23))
 (segment (start 163.575 96.54) (end 165.08 96.54) (width 0.25) (layer "F.Cu") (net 23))
 (segment (start 165.08 96.54) (end 175.26 86.36) (width 0.25) (layer "F.Cu") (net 23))
 (segment (start 175.26 86.36) (end 175.26 55.88) (width 0.25) (layer "F.Cu") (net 23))
 (segment (start 185.42 60.96) (end 192.62 60.96) (width 0.25) (layer "F.Cu") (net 23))
 (via (at 175.26 55.88) (size 0.8) (drill 0.4) (layers "F.Cu" "B.Cu") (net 23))
 (via (at 175.26 55.88) (size 0.8) (drill 0.4) (layers "F.Cu" "B.Cu") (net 23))
 (via (at 175.26 55.88) (size 0.8) (drill 0.4) (layers "F.Cu" "B.Cu") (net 23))
 (segment (start 175.26 55.88) (end 180.34 55.88) (width 0.25) (layer "B.Cu") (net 23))
 (segment (start 180.34 55.88) (end 184.268719 59.808719) (width 0.25) (layer "B.Cu") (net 23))
 (segment (start 191.21 99.35) (end 194.87 99.35) (width 0.25) (layer "F.Cu") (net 2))
 (segment (start 186.13 104.43) (end 191.21 99.35) (width 0.25) (layer "F.Cu") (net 2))
 (segment (start 165.08 94) (end 167.64 91.44) (width 0.25) (layer "F.Cu") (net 2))
 (segment (start 163.575 94) (end 165.08 94) (width 0.25) (layer "F.Cu") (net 2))
 (via (at 167.64 91.44) (size 0.8) (drill 0.4) (layers "F.Cu" "B.Cu") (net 2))
 (via (at 167.64 91.44) (size 0.8) (drill 0.4) (layers "F.Cu" "B.Cu") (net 2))
 (segment (start 173.14 91.44) (end 186.13 104.43) (width 0.25) (layer "B.Cu") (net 2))
 (segment (start 167.64 91.44) (end 173.14 91.44) (width 0.25) (layer "B.Cu") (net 2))
 (segment (start 163.575 91.46) (end 160.04 91.46) (width 0.25) (layer "F.Cu") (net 24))
 (segment (start 160.04 91.46) (end 160.02 91.44) (width 0.25) (layer "F.Cu") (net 24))
 (via (at 160.02 91.44) (size 0.8) (drill 0.4) (layers "F.Cu" "B.Cu") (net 24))
 (segment (start 160.02 91.44) (end 158.875 92.585) (width 0.25) (layer "B.Cu") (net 24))
 (segment (start 122.595 98.135) (end 117.001167 98.135) (width 0.25) (layer "B.Cu") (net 24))
 (segment (start 158.875 92.585) (end 128.145 92.585) (width 0.25) (layer "B.Cu") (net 24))
 (segment (start 116.225 89.515) (end 116.84 88.9) (width 0.25) (layer "B.Cu") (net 24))
 (segment (start 117.001167 98.135) (end 116.225 97.358833) (width 0.25) (layer "B.Cu") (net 24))
 (segment (start 128.145 92.585) (end 122.595 98.135) (width 0.25) (layer "B.Cu") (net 24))
 (segment (start 116.225 97.358833) (end 116.225 89.515) (width 0.25) (layer "B.Cu") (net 24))
 (segment (start 167.62 88.92) (end 167.64 88.9) (width 0.25) (layer "F.Cu") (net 25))
 (segment (start 163.575 88.92) (end 167.62 88.92) (width 0.25) (layer "F.Cu") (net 25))
 (via (at 167.64 88.9) (size 0.8) (drill 0.4) (layers "F.Cu" "B.Cu") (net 25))
 (via (at 167.64 88.9) (size 0.8) (drill 0.4) (layers "F.Cu" "B.Cu") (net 25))
 (segment (start 167.64 88.9) (end 168.375 88.165) (width 0.25) (layer "B.Cu") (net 25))
 (segment (start 197.605 87.965) (end 198.83 89.19) (width 0.25) (layer "B.Cu") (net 25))
 (segment (start 194.845 88.165) (end 195.045 87.965) (width 0.25) (layer "B.Cu") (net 25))
 (segment (start 168.375 88.165) (end 194.845 88.165) (width 0.25) (layer "B.Cu") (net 25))
 (segment (start 195.045 87.965) (end 197.605 87.965) (width 0.25) (layer "B.Cu") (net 25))
 (segment (start 145.885 105.575) (end 148.135 107.825) (width 0.25) (layer "B.Cu") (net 27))
 (segment (start 164.040991 107.825) (end 164.7 107.165991) (width 0.25) (layer "B.Cu") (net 27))
 (segment (start 164.7 107.165991) (end 164.7 84.965) (width 0.25) (layer "B.Cu") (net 27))
 (segment (start 148.135 107.825) (end 164.040991 107.825) (width 0.25) (layer "B.Cu") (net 27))
 (segment (start 128.525 105.575) (end 145.885 105.575) (width 0.25) (layer "B.Cu") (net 27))
 (segment (start 164.7 84.965) (end 163.575 83.84) (width 0.25) (layer "B.Cu") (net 27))
 (segment (start 117.55 116.55) (end 128.525 105.575) (width 0.25) (layer "B.Cu") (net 27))
 (segment (start 140.965 58.69) (end 163.575 81.3) (width 0.25) (layer "B.Cu") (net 6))
 (segment (start 140.965 37.395) (end 140.965 58.69) (width 0.25) (layer "B.Cu") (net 6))
 (segment (start 125.775 90.125) (end 115.525 90.125) (width 0.25) (layer "F.Cu") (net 29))
 (segment (start 115.525 90.125) (end 114.3 88.9) (width 0.25) (layer "F.Cu") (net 29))
 (segment (start 127 88.9) (end 125.775 90.125) (width 0.25) (layer "F.Cu") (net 29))
 (segment (start 186.13 89.19) (end 196.29 89.19) (width 0.25) (layer "F.Cu") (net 28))
 (segment (start 138.425 37.395) (end 138.425 44.455) (width 0.25) (layer "F.Cu") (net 1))
 (segment (start 147.32 36.12) (end 146.045 37.395) (width 0.25) (layer "F.Cu") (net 1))
 (segment (start 149.86 85.365) (end 149.86 86.36) (width 0.25) (layer "F.Cu") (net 1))
 (segment (start 143.255 78.76) (end 149.86 85.365) (width 0.25) (layer "F.Cu") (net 1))
 (segment (start 180.34 60.96) (end 180.34 45.72) (width 0.25) (layer "F.Cu") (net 1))
 (segment (start 132.08 88.9) (end 132.08 101.24) (width 0.25) (layer "F.Cu") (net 1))
 (segment (start 156.91 35.56) (end 154.94 35.56) (width 0.25) (layer "F.Cu") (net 1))
 (segment (start 187.95 106.25) (end 182.87 106.25) (width 0.25) (layer "F.Cu") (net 1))
 (segment (start 158.745 37.395) (end 156.91 35.56) (width 0.25) (layer "F.Cu") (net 1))
 (segment (start 129.54 53.34) (end 149.86 53.34) (width 0.25) (layer "F.Cu") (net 1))
 (segment (start 139.72 109.24) (end 132.08 101.6) (width 0.25) (layer "F.Cu") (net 1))
 (segment (start 153.665 37.395) (end 151.83 35.56) (width 0.25) (layer "F.Cu") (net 1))
 (segment (start 139.7 36.12) (end 138.425 37.395) (width 0.25) (layer "F.Cu") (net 1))
 (segment (start 144.21 35.56) (end 139.7 35.56) (width 0.25) (layer "F.Cu") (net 1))
 (segment (start 138.425 44.455) (end 129.54 53.34) (width 0.25) (layer "F.Cu") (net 1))
 (segment (start 154.94 36.12) (end 153.665 37.395) (width 0.25) (layer "F.Cu") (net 1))
 (segment (start 154.94 35.56) (end 154.94 36.12) (width 0.25) (layer "F.Cu") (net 1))
 (segment (start 170.84 36.22) (end 159.92 36.22) (width 0.25) (layer "F.Cu") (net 1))
 (segment (start 151.83 35.56) (end 147.32 35.56) (width 0.25) (layer "F.Cu") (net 1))
 (segment (start 132.08 88.9) (end 132.08 55.88) (width 0.25) (layer "F.Cu") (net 1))
 (segment (start 147.32 35.56) (end 147.32 36.12) (width 0.25) (layer "F.Cu") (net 1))
 (segment (start 181.05 89.19) (end 181.05 61.67) (width 0.25) (layer "F.Cu") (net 1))
 (segment (start 121.27 112.05) (end 117.55 112.05) (width 0.25) (layer "F.Cu") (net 1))
 (segment (start 146.045 37.395) (end 144.21 35.56) (width 0.25) (layer "F.Cu") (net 1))
 (segment (start 132.08 101.24) (end 121.27 112.05) (width 0.25) (layer "F.Cu") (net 1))
 (segment (start 182.87 106.25) (end 181.05 104.43) (width 0.25) (layer "F.Cu") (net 1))
 (segment (start 180.34 45.72) (end 170.84 36.22) (width 0.25) (layer "F.Cu") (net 1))
 (segment (start 143.255 109.24) (end 139.72 109.24) (width 0.25) (layer "F.Cu") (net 1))
 (segment (start 159.92 36.22) (end 158.745 37.395) (width 0.25) (layer "F.Cu") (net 1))
 (segment (start 181.05 61.67) (end 180.34 60.96) (width 0.25) (layer "F.Cu") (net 1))
 (segment (start 198.83 117.13) (end 187.95 106.25) (width 0.25) (layer "F.Cu") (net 1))
 (segment (start 139.7 35.56) (end 139.7 36.12) (width 0.25) (layer "F.Cu") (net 1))
 (segment (start 181.05 104.43) (end 181.05 89.19) (width 0.25) (layer "F.Cu") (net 1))
 (segment (start 132.08 55.88) (end 129.54 53.34) (width 0.25) (layer "F.Cu") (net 1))
 (via (at 149.86 86.36) (size 0.8) (drill 0.4) (layers "F.Cu" "B.Cu") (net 1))
 (via (at 149.86 86.36) (size 0.8) (drill 0.4) (layers "F.Cu" "B.Cu") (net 1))
 (segment (start 146.175 90.045) (end 133.225 90.045) (width 0.25) (layer "B.Cu") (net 1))
 (segment (start 133.225 90.045) (end 132.08 88.9) (width 0.25) (layer "B.Cu") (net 1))
 (segment (start 149.86 86.36) (end 146.175 90.045) (width 0.25) (layer "B.Cu") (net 1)))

